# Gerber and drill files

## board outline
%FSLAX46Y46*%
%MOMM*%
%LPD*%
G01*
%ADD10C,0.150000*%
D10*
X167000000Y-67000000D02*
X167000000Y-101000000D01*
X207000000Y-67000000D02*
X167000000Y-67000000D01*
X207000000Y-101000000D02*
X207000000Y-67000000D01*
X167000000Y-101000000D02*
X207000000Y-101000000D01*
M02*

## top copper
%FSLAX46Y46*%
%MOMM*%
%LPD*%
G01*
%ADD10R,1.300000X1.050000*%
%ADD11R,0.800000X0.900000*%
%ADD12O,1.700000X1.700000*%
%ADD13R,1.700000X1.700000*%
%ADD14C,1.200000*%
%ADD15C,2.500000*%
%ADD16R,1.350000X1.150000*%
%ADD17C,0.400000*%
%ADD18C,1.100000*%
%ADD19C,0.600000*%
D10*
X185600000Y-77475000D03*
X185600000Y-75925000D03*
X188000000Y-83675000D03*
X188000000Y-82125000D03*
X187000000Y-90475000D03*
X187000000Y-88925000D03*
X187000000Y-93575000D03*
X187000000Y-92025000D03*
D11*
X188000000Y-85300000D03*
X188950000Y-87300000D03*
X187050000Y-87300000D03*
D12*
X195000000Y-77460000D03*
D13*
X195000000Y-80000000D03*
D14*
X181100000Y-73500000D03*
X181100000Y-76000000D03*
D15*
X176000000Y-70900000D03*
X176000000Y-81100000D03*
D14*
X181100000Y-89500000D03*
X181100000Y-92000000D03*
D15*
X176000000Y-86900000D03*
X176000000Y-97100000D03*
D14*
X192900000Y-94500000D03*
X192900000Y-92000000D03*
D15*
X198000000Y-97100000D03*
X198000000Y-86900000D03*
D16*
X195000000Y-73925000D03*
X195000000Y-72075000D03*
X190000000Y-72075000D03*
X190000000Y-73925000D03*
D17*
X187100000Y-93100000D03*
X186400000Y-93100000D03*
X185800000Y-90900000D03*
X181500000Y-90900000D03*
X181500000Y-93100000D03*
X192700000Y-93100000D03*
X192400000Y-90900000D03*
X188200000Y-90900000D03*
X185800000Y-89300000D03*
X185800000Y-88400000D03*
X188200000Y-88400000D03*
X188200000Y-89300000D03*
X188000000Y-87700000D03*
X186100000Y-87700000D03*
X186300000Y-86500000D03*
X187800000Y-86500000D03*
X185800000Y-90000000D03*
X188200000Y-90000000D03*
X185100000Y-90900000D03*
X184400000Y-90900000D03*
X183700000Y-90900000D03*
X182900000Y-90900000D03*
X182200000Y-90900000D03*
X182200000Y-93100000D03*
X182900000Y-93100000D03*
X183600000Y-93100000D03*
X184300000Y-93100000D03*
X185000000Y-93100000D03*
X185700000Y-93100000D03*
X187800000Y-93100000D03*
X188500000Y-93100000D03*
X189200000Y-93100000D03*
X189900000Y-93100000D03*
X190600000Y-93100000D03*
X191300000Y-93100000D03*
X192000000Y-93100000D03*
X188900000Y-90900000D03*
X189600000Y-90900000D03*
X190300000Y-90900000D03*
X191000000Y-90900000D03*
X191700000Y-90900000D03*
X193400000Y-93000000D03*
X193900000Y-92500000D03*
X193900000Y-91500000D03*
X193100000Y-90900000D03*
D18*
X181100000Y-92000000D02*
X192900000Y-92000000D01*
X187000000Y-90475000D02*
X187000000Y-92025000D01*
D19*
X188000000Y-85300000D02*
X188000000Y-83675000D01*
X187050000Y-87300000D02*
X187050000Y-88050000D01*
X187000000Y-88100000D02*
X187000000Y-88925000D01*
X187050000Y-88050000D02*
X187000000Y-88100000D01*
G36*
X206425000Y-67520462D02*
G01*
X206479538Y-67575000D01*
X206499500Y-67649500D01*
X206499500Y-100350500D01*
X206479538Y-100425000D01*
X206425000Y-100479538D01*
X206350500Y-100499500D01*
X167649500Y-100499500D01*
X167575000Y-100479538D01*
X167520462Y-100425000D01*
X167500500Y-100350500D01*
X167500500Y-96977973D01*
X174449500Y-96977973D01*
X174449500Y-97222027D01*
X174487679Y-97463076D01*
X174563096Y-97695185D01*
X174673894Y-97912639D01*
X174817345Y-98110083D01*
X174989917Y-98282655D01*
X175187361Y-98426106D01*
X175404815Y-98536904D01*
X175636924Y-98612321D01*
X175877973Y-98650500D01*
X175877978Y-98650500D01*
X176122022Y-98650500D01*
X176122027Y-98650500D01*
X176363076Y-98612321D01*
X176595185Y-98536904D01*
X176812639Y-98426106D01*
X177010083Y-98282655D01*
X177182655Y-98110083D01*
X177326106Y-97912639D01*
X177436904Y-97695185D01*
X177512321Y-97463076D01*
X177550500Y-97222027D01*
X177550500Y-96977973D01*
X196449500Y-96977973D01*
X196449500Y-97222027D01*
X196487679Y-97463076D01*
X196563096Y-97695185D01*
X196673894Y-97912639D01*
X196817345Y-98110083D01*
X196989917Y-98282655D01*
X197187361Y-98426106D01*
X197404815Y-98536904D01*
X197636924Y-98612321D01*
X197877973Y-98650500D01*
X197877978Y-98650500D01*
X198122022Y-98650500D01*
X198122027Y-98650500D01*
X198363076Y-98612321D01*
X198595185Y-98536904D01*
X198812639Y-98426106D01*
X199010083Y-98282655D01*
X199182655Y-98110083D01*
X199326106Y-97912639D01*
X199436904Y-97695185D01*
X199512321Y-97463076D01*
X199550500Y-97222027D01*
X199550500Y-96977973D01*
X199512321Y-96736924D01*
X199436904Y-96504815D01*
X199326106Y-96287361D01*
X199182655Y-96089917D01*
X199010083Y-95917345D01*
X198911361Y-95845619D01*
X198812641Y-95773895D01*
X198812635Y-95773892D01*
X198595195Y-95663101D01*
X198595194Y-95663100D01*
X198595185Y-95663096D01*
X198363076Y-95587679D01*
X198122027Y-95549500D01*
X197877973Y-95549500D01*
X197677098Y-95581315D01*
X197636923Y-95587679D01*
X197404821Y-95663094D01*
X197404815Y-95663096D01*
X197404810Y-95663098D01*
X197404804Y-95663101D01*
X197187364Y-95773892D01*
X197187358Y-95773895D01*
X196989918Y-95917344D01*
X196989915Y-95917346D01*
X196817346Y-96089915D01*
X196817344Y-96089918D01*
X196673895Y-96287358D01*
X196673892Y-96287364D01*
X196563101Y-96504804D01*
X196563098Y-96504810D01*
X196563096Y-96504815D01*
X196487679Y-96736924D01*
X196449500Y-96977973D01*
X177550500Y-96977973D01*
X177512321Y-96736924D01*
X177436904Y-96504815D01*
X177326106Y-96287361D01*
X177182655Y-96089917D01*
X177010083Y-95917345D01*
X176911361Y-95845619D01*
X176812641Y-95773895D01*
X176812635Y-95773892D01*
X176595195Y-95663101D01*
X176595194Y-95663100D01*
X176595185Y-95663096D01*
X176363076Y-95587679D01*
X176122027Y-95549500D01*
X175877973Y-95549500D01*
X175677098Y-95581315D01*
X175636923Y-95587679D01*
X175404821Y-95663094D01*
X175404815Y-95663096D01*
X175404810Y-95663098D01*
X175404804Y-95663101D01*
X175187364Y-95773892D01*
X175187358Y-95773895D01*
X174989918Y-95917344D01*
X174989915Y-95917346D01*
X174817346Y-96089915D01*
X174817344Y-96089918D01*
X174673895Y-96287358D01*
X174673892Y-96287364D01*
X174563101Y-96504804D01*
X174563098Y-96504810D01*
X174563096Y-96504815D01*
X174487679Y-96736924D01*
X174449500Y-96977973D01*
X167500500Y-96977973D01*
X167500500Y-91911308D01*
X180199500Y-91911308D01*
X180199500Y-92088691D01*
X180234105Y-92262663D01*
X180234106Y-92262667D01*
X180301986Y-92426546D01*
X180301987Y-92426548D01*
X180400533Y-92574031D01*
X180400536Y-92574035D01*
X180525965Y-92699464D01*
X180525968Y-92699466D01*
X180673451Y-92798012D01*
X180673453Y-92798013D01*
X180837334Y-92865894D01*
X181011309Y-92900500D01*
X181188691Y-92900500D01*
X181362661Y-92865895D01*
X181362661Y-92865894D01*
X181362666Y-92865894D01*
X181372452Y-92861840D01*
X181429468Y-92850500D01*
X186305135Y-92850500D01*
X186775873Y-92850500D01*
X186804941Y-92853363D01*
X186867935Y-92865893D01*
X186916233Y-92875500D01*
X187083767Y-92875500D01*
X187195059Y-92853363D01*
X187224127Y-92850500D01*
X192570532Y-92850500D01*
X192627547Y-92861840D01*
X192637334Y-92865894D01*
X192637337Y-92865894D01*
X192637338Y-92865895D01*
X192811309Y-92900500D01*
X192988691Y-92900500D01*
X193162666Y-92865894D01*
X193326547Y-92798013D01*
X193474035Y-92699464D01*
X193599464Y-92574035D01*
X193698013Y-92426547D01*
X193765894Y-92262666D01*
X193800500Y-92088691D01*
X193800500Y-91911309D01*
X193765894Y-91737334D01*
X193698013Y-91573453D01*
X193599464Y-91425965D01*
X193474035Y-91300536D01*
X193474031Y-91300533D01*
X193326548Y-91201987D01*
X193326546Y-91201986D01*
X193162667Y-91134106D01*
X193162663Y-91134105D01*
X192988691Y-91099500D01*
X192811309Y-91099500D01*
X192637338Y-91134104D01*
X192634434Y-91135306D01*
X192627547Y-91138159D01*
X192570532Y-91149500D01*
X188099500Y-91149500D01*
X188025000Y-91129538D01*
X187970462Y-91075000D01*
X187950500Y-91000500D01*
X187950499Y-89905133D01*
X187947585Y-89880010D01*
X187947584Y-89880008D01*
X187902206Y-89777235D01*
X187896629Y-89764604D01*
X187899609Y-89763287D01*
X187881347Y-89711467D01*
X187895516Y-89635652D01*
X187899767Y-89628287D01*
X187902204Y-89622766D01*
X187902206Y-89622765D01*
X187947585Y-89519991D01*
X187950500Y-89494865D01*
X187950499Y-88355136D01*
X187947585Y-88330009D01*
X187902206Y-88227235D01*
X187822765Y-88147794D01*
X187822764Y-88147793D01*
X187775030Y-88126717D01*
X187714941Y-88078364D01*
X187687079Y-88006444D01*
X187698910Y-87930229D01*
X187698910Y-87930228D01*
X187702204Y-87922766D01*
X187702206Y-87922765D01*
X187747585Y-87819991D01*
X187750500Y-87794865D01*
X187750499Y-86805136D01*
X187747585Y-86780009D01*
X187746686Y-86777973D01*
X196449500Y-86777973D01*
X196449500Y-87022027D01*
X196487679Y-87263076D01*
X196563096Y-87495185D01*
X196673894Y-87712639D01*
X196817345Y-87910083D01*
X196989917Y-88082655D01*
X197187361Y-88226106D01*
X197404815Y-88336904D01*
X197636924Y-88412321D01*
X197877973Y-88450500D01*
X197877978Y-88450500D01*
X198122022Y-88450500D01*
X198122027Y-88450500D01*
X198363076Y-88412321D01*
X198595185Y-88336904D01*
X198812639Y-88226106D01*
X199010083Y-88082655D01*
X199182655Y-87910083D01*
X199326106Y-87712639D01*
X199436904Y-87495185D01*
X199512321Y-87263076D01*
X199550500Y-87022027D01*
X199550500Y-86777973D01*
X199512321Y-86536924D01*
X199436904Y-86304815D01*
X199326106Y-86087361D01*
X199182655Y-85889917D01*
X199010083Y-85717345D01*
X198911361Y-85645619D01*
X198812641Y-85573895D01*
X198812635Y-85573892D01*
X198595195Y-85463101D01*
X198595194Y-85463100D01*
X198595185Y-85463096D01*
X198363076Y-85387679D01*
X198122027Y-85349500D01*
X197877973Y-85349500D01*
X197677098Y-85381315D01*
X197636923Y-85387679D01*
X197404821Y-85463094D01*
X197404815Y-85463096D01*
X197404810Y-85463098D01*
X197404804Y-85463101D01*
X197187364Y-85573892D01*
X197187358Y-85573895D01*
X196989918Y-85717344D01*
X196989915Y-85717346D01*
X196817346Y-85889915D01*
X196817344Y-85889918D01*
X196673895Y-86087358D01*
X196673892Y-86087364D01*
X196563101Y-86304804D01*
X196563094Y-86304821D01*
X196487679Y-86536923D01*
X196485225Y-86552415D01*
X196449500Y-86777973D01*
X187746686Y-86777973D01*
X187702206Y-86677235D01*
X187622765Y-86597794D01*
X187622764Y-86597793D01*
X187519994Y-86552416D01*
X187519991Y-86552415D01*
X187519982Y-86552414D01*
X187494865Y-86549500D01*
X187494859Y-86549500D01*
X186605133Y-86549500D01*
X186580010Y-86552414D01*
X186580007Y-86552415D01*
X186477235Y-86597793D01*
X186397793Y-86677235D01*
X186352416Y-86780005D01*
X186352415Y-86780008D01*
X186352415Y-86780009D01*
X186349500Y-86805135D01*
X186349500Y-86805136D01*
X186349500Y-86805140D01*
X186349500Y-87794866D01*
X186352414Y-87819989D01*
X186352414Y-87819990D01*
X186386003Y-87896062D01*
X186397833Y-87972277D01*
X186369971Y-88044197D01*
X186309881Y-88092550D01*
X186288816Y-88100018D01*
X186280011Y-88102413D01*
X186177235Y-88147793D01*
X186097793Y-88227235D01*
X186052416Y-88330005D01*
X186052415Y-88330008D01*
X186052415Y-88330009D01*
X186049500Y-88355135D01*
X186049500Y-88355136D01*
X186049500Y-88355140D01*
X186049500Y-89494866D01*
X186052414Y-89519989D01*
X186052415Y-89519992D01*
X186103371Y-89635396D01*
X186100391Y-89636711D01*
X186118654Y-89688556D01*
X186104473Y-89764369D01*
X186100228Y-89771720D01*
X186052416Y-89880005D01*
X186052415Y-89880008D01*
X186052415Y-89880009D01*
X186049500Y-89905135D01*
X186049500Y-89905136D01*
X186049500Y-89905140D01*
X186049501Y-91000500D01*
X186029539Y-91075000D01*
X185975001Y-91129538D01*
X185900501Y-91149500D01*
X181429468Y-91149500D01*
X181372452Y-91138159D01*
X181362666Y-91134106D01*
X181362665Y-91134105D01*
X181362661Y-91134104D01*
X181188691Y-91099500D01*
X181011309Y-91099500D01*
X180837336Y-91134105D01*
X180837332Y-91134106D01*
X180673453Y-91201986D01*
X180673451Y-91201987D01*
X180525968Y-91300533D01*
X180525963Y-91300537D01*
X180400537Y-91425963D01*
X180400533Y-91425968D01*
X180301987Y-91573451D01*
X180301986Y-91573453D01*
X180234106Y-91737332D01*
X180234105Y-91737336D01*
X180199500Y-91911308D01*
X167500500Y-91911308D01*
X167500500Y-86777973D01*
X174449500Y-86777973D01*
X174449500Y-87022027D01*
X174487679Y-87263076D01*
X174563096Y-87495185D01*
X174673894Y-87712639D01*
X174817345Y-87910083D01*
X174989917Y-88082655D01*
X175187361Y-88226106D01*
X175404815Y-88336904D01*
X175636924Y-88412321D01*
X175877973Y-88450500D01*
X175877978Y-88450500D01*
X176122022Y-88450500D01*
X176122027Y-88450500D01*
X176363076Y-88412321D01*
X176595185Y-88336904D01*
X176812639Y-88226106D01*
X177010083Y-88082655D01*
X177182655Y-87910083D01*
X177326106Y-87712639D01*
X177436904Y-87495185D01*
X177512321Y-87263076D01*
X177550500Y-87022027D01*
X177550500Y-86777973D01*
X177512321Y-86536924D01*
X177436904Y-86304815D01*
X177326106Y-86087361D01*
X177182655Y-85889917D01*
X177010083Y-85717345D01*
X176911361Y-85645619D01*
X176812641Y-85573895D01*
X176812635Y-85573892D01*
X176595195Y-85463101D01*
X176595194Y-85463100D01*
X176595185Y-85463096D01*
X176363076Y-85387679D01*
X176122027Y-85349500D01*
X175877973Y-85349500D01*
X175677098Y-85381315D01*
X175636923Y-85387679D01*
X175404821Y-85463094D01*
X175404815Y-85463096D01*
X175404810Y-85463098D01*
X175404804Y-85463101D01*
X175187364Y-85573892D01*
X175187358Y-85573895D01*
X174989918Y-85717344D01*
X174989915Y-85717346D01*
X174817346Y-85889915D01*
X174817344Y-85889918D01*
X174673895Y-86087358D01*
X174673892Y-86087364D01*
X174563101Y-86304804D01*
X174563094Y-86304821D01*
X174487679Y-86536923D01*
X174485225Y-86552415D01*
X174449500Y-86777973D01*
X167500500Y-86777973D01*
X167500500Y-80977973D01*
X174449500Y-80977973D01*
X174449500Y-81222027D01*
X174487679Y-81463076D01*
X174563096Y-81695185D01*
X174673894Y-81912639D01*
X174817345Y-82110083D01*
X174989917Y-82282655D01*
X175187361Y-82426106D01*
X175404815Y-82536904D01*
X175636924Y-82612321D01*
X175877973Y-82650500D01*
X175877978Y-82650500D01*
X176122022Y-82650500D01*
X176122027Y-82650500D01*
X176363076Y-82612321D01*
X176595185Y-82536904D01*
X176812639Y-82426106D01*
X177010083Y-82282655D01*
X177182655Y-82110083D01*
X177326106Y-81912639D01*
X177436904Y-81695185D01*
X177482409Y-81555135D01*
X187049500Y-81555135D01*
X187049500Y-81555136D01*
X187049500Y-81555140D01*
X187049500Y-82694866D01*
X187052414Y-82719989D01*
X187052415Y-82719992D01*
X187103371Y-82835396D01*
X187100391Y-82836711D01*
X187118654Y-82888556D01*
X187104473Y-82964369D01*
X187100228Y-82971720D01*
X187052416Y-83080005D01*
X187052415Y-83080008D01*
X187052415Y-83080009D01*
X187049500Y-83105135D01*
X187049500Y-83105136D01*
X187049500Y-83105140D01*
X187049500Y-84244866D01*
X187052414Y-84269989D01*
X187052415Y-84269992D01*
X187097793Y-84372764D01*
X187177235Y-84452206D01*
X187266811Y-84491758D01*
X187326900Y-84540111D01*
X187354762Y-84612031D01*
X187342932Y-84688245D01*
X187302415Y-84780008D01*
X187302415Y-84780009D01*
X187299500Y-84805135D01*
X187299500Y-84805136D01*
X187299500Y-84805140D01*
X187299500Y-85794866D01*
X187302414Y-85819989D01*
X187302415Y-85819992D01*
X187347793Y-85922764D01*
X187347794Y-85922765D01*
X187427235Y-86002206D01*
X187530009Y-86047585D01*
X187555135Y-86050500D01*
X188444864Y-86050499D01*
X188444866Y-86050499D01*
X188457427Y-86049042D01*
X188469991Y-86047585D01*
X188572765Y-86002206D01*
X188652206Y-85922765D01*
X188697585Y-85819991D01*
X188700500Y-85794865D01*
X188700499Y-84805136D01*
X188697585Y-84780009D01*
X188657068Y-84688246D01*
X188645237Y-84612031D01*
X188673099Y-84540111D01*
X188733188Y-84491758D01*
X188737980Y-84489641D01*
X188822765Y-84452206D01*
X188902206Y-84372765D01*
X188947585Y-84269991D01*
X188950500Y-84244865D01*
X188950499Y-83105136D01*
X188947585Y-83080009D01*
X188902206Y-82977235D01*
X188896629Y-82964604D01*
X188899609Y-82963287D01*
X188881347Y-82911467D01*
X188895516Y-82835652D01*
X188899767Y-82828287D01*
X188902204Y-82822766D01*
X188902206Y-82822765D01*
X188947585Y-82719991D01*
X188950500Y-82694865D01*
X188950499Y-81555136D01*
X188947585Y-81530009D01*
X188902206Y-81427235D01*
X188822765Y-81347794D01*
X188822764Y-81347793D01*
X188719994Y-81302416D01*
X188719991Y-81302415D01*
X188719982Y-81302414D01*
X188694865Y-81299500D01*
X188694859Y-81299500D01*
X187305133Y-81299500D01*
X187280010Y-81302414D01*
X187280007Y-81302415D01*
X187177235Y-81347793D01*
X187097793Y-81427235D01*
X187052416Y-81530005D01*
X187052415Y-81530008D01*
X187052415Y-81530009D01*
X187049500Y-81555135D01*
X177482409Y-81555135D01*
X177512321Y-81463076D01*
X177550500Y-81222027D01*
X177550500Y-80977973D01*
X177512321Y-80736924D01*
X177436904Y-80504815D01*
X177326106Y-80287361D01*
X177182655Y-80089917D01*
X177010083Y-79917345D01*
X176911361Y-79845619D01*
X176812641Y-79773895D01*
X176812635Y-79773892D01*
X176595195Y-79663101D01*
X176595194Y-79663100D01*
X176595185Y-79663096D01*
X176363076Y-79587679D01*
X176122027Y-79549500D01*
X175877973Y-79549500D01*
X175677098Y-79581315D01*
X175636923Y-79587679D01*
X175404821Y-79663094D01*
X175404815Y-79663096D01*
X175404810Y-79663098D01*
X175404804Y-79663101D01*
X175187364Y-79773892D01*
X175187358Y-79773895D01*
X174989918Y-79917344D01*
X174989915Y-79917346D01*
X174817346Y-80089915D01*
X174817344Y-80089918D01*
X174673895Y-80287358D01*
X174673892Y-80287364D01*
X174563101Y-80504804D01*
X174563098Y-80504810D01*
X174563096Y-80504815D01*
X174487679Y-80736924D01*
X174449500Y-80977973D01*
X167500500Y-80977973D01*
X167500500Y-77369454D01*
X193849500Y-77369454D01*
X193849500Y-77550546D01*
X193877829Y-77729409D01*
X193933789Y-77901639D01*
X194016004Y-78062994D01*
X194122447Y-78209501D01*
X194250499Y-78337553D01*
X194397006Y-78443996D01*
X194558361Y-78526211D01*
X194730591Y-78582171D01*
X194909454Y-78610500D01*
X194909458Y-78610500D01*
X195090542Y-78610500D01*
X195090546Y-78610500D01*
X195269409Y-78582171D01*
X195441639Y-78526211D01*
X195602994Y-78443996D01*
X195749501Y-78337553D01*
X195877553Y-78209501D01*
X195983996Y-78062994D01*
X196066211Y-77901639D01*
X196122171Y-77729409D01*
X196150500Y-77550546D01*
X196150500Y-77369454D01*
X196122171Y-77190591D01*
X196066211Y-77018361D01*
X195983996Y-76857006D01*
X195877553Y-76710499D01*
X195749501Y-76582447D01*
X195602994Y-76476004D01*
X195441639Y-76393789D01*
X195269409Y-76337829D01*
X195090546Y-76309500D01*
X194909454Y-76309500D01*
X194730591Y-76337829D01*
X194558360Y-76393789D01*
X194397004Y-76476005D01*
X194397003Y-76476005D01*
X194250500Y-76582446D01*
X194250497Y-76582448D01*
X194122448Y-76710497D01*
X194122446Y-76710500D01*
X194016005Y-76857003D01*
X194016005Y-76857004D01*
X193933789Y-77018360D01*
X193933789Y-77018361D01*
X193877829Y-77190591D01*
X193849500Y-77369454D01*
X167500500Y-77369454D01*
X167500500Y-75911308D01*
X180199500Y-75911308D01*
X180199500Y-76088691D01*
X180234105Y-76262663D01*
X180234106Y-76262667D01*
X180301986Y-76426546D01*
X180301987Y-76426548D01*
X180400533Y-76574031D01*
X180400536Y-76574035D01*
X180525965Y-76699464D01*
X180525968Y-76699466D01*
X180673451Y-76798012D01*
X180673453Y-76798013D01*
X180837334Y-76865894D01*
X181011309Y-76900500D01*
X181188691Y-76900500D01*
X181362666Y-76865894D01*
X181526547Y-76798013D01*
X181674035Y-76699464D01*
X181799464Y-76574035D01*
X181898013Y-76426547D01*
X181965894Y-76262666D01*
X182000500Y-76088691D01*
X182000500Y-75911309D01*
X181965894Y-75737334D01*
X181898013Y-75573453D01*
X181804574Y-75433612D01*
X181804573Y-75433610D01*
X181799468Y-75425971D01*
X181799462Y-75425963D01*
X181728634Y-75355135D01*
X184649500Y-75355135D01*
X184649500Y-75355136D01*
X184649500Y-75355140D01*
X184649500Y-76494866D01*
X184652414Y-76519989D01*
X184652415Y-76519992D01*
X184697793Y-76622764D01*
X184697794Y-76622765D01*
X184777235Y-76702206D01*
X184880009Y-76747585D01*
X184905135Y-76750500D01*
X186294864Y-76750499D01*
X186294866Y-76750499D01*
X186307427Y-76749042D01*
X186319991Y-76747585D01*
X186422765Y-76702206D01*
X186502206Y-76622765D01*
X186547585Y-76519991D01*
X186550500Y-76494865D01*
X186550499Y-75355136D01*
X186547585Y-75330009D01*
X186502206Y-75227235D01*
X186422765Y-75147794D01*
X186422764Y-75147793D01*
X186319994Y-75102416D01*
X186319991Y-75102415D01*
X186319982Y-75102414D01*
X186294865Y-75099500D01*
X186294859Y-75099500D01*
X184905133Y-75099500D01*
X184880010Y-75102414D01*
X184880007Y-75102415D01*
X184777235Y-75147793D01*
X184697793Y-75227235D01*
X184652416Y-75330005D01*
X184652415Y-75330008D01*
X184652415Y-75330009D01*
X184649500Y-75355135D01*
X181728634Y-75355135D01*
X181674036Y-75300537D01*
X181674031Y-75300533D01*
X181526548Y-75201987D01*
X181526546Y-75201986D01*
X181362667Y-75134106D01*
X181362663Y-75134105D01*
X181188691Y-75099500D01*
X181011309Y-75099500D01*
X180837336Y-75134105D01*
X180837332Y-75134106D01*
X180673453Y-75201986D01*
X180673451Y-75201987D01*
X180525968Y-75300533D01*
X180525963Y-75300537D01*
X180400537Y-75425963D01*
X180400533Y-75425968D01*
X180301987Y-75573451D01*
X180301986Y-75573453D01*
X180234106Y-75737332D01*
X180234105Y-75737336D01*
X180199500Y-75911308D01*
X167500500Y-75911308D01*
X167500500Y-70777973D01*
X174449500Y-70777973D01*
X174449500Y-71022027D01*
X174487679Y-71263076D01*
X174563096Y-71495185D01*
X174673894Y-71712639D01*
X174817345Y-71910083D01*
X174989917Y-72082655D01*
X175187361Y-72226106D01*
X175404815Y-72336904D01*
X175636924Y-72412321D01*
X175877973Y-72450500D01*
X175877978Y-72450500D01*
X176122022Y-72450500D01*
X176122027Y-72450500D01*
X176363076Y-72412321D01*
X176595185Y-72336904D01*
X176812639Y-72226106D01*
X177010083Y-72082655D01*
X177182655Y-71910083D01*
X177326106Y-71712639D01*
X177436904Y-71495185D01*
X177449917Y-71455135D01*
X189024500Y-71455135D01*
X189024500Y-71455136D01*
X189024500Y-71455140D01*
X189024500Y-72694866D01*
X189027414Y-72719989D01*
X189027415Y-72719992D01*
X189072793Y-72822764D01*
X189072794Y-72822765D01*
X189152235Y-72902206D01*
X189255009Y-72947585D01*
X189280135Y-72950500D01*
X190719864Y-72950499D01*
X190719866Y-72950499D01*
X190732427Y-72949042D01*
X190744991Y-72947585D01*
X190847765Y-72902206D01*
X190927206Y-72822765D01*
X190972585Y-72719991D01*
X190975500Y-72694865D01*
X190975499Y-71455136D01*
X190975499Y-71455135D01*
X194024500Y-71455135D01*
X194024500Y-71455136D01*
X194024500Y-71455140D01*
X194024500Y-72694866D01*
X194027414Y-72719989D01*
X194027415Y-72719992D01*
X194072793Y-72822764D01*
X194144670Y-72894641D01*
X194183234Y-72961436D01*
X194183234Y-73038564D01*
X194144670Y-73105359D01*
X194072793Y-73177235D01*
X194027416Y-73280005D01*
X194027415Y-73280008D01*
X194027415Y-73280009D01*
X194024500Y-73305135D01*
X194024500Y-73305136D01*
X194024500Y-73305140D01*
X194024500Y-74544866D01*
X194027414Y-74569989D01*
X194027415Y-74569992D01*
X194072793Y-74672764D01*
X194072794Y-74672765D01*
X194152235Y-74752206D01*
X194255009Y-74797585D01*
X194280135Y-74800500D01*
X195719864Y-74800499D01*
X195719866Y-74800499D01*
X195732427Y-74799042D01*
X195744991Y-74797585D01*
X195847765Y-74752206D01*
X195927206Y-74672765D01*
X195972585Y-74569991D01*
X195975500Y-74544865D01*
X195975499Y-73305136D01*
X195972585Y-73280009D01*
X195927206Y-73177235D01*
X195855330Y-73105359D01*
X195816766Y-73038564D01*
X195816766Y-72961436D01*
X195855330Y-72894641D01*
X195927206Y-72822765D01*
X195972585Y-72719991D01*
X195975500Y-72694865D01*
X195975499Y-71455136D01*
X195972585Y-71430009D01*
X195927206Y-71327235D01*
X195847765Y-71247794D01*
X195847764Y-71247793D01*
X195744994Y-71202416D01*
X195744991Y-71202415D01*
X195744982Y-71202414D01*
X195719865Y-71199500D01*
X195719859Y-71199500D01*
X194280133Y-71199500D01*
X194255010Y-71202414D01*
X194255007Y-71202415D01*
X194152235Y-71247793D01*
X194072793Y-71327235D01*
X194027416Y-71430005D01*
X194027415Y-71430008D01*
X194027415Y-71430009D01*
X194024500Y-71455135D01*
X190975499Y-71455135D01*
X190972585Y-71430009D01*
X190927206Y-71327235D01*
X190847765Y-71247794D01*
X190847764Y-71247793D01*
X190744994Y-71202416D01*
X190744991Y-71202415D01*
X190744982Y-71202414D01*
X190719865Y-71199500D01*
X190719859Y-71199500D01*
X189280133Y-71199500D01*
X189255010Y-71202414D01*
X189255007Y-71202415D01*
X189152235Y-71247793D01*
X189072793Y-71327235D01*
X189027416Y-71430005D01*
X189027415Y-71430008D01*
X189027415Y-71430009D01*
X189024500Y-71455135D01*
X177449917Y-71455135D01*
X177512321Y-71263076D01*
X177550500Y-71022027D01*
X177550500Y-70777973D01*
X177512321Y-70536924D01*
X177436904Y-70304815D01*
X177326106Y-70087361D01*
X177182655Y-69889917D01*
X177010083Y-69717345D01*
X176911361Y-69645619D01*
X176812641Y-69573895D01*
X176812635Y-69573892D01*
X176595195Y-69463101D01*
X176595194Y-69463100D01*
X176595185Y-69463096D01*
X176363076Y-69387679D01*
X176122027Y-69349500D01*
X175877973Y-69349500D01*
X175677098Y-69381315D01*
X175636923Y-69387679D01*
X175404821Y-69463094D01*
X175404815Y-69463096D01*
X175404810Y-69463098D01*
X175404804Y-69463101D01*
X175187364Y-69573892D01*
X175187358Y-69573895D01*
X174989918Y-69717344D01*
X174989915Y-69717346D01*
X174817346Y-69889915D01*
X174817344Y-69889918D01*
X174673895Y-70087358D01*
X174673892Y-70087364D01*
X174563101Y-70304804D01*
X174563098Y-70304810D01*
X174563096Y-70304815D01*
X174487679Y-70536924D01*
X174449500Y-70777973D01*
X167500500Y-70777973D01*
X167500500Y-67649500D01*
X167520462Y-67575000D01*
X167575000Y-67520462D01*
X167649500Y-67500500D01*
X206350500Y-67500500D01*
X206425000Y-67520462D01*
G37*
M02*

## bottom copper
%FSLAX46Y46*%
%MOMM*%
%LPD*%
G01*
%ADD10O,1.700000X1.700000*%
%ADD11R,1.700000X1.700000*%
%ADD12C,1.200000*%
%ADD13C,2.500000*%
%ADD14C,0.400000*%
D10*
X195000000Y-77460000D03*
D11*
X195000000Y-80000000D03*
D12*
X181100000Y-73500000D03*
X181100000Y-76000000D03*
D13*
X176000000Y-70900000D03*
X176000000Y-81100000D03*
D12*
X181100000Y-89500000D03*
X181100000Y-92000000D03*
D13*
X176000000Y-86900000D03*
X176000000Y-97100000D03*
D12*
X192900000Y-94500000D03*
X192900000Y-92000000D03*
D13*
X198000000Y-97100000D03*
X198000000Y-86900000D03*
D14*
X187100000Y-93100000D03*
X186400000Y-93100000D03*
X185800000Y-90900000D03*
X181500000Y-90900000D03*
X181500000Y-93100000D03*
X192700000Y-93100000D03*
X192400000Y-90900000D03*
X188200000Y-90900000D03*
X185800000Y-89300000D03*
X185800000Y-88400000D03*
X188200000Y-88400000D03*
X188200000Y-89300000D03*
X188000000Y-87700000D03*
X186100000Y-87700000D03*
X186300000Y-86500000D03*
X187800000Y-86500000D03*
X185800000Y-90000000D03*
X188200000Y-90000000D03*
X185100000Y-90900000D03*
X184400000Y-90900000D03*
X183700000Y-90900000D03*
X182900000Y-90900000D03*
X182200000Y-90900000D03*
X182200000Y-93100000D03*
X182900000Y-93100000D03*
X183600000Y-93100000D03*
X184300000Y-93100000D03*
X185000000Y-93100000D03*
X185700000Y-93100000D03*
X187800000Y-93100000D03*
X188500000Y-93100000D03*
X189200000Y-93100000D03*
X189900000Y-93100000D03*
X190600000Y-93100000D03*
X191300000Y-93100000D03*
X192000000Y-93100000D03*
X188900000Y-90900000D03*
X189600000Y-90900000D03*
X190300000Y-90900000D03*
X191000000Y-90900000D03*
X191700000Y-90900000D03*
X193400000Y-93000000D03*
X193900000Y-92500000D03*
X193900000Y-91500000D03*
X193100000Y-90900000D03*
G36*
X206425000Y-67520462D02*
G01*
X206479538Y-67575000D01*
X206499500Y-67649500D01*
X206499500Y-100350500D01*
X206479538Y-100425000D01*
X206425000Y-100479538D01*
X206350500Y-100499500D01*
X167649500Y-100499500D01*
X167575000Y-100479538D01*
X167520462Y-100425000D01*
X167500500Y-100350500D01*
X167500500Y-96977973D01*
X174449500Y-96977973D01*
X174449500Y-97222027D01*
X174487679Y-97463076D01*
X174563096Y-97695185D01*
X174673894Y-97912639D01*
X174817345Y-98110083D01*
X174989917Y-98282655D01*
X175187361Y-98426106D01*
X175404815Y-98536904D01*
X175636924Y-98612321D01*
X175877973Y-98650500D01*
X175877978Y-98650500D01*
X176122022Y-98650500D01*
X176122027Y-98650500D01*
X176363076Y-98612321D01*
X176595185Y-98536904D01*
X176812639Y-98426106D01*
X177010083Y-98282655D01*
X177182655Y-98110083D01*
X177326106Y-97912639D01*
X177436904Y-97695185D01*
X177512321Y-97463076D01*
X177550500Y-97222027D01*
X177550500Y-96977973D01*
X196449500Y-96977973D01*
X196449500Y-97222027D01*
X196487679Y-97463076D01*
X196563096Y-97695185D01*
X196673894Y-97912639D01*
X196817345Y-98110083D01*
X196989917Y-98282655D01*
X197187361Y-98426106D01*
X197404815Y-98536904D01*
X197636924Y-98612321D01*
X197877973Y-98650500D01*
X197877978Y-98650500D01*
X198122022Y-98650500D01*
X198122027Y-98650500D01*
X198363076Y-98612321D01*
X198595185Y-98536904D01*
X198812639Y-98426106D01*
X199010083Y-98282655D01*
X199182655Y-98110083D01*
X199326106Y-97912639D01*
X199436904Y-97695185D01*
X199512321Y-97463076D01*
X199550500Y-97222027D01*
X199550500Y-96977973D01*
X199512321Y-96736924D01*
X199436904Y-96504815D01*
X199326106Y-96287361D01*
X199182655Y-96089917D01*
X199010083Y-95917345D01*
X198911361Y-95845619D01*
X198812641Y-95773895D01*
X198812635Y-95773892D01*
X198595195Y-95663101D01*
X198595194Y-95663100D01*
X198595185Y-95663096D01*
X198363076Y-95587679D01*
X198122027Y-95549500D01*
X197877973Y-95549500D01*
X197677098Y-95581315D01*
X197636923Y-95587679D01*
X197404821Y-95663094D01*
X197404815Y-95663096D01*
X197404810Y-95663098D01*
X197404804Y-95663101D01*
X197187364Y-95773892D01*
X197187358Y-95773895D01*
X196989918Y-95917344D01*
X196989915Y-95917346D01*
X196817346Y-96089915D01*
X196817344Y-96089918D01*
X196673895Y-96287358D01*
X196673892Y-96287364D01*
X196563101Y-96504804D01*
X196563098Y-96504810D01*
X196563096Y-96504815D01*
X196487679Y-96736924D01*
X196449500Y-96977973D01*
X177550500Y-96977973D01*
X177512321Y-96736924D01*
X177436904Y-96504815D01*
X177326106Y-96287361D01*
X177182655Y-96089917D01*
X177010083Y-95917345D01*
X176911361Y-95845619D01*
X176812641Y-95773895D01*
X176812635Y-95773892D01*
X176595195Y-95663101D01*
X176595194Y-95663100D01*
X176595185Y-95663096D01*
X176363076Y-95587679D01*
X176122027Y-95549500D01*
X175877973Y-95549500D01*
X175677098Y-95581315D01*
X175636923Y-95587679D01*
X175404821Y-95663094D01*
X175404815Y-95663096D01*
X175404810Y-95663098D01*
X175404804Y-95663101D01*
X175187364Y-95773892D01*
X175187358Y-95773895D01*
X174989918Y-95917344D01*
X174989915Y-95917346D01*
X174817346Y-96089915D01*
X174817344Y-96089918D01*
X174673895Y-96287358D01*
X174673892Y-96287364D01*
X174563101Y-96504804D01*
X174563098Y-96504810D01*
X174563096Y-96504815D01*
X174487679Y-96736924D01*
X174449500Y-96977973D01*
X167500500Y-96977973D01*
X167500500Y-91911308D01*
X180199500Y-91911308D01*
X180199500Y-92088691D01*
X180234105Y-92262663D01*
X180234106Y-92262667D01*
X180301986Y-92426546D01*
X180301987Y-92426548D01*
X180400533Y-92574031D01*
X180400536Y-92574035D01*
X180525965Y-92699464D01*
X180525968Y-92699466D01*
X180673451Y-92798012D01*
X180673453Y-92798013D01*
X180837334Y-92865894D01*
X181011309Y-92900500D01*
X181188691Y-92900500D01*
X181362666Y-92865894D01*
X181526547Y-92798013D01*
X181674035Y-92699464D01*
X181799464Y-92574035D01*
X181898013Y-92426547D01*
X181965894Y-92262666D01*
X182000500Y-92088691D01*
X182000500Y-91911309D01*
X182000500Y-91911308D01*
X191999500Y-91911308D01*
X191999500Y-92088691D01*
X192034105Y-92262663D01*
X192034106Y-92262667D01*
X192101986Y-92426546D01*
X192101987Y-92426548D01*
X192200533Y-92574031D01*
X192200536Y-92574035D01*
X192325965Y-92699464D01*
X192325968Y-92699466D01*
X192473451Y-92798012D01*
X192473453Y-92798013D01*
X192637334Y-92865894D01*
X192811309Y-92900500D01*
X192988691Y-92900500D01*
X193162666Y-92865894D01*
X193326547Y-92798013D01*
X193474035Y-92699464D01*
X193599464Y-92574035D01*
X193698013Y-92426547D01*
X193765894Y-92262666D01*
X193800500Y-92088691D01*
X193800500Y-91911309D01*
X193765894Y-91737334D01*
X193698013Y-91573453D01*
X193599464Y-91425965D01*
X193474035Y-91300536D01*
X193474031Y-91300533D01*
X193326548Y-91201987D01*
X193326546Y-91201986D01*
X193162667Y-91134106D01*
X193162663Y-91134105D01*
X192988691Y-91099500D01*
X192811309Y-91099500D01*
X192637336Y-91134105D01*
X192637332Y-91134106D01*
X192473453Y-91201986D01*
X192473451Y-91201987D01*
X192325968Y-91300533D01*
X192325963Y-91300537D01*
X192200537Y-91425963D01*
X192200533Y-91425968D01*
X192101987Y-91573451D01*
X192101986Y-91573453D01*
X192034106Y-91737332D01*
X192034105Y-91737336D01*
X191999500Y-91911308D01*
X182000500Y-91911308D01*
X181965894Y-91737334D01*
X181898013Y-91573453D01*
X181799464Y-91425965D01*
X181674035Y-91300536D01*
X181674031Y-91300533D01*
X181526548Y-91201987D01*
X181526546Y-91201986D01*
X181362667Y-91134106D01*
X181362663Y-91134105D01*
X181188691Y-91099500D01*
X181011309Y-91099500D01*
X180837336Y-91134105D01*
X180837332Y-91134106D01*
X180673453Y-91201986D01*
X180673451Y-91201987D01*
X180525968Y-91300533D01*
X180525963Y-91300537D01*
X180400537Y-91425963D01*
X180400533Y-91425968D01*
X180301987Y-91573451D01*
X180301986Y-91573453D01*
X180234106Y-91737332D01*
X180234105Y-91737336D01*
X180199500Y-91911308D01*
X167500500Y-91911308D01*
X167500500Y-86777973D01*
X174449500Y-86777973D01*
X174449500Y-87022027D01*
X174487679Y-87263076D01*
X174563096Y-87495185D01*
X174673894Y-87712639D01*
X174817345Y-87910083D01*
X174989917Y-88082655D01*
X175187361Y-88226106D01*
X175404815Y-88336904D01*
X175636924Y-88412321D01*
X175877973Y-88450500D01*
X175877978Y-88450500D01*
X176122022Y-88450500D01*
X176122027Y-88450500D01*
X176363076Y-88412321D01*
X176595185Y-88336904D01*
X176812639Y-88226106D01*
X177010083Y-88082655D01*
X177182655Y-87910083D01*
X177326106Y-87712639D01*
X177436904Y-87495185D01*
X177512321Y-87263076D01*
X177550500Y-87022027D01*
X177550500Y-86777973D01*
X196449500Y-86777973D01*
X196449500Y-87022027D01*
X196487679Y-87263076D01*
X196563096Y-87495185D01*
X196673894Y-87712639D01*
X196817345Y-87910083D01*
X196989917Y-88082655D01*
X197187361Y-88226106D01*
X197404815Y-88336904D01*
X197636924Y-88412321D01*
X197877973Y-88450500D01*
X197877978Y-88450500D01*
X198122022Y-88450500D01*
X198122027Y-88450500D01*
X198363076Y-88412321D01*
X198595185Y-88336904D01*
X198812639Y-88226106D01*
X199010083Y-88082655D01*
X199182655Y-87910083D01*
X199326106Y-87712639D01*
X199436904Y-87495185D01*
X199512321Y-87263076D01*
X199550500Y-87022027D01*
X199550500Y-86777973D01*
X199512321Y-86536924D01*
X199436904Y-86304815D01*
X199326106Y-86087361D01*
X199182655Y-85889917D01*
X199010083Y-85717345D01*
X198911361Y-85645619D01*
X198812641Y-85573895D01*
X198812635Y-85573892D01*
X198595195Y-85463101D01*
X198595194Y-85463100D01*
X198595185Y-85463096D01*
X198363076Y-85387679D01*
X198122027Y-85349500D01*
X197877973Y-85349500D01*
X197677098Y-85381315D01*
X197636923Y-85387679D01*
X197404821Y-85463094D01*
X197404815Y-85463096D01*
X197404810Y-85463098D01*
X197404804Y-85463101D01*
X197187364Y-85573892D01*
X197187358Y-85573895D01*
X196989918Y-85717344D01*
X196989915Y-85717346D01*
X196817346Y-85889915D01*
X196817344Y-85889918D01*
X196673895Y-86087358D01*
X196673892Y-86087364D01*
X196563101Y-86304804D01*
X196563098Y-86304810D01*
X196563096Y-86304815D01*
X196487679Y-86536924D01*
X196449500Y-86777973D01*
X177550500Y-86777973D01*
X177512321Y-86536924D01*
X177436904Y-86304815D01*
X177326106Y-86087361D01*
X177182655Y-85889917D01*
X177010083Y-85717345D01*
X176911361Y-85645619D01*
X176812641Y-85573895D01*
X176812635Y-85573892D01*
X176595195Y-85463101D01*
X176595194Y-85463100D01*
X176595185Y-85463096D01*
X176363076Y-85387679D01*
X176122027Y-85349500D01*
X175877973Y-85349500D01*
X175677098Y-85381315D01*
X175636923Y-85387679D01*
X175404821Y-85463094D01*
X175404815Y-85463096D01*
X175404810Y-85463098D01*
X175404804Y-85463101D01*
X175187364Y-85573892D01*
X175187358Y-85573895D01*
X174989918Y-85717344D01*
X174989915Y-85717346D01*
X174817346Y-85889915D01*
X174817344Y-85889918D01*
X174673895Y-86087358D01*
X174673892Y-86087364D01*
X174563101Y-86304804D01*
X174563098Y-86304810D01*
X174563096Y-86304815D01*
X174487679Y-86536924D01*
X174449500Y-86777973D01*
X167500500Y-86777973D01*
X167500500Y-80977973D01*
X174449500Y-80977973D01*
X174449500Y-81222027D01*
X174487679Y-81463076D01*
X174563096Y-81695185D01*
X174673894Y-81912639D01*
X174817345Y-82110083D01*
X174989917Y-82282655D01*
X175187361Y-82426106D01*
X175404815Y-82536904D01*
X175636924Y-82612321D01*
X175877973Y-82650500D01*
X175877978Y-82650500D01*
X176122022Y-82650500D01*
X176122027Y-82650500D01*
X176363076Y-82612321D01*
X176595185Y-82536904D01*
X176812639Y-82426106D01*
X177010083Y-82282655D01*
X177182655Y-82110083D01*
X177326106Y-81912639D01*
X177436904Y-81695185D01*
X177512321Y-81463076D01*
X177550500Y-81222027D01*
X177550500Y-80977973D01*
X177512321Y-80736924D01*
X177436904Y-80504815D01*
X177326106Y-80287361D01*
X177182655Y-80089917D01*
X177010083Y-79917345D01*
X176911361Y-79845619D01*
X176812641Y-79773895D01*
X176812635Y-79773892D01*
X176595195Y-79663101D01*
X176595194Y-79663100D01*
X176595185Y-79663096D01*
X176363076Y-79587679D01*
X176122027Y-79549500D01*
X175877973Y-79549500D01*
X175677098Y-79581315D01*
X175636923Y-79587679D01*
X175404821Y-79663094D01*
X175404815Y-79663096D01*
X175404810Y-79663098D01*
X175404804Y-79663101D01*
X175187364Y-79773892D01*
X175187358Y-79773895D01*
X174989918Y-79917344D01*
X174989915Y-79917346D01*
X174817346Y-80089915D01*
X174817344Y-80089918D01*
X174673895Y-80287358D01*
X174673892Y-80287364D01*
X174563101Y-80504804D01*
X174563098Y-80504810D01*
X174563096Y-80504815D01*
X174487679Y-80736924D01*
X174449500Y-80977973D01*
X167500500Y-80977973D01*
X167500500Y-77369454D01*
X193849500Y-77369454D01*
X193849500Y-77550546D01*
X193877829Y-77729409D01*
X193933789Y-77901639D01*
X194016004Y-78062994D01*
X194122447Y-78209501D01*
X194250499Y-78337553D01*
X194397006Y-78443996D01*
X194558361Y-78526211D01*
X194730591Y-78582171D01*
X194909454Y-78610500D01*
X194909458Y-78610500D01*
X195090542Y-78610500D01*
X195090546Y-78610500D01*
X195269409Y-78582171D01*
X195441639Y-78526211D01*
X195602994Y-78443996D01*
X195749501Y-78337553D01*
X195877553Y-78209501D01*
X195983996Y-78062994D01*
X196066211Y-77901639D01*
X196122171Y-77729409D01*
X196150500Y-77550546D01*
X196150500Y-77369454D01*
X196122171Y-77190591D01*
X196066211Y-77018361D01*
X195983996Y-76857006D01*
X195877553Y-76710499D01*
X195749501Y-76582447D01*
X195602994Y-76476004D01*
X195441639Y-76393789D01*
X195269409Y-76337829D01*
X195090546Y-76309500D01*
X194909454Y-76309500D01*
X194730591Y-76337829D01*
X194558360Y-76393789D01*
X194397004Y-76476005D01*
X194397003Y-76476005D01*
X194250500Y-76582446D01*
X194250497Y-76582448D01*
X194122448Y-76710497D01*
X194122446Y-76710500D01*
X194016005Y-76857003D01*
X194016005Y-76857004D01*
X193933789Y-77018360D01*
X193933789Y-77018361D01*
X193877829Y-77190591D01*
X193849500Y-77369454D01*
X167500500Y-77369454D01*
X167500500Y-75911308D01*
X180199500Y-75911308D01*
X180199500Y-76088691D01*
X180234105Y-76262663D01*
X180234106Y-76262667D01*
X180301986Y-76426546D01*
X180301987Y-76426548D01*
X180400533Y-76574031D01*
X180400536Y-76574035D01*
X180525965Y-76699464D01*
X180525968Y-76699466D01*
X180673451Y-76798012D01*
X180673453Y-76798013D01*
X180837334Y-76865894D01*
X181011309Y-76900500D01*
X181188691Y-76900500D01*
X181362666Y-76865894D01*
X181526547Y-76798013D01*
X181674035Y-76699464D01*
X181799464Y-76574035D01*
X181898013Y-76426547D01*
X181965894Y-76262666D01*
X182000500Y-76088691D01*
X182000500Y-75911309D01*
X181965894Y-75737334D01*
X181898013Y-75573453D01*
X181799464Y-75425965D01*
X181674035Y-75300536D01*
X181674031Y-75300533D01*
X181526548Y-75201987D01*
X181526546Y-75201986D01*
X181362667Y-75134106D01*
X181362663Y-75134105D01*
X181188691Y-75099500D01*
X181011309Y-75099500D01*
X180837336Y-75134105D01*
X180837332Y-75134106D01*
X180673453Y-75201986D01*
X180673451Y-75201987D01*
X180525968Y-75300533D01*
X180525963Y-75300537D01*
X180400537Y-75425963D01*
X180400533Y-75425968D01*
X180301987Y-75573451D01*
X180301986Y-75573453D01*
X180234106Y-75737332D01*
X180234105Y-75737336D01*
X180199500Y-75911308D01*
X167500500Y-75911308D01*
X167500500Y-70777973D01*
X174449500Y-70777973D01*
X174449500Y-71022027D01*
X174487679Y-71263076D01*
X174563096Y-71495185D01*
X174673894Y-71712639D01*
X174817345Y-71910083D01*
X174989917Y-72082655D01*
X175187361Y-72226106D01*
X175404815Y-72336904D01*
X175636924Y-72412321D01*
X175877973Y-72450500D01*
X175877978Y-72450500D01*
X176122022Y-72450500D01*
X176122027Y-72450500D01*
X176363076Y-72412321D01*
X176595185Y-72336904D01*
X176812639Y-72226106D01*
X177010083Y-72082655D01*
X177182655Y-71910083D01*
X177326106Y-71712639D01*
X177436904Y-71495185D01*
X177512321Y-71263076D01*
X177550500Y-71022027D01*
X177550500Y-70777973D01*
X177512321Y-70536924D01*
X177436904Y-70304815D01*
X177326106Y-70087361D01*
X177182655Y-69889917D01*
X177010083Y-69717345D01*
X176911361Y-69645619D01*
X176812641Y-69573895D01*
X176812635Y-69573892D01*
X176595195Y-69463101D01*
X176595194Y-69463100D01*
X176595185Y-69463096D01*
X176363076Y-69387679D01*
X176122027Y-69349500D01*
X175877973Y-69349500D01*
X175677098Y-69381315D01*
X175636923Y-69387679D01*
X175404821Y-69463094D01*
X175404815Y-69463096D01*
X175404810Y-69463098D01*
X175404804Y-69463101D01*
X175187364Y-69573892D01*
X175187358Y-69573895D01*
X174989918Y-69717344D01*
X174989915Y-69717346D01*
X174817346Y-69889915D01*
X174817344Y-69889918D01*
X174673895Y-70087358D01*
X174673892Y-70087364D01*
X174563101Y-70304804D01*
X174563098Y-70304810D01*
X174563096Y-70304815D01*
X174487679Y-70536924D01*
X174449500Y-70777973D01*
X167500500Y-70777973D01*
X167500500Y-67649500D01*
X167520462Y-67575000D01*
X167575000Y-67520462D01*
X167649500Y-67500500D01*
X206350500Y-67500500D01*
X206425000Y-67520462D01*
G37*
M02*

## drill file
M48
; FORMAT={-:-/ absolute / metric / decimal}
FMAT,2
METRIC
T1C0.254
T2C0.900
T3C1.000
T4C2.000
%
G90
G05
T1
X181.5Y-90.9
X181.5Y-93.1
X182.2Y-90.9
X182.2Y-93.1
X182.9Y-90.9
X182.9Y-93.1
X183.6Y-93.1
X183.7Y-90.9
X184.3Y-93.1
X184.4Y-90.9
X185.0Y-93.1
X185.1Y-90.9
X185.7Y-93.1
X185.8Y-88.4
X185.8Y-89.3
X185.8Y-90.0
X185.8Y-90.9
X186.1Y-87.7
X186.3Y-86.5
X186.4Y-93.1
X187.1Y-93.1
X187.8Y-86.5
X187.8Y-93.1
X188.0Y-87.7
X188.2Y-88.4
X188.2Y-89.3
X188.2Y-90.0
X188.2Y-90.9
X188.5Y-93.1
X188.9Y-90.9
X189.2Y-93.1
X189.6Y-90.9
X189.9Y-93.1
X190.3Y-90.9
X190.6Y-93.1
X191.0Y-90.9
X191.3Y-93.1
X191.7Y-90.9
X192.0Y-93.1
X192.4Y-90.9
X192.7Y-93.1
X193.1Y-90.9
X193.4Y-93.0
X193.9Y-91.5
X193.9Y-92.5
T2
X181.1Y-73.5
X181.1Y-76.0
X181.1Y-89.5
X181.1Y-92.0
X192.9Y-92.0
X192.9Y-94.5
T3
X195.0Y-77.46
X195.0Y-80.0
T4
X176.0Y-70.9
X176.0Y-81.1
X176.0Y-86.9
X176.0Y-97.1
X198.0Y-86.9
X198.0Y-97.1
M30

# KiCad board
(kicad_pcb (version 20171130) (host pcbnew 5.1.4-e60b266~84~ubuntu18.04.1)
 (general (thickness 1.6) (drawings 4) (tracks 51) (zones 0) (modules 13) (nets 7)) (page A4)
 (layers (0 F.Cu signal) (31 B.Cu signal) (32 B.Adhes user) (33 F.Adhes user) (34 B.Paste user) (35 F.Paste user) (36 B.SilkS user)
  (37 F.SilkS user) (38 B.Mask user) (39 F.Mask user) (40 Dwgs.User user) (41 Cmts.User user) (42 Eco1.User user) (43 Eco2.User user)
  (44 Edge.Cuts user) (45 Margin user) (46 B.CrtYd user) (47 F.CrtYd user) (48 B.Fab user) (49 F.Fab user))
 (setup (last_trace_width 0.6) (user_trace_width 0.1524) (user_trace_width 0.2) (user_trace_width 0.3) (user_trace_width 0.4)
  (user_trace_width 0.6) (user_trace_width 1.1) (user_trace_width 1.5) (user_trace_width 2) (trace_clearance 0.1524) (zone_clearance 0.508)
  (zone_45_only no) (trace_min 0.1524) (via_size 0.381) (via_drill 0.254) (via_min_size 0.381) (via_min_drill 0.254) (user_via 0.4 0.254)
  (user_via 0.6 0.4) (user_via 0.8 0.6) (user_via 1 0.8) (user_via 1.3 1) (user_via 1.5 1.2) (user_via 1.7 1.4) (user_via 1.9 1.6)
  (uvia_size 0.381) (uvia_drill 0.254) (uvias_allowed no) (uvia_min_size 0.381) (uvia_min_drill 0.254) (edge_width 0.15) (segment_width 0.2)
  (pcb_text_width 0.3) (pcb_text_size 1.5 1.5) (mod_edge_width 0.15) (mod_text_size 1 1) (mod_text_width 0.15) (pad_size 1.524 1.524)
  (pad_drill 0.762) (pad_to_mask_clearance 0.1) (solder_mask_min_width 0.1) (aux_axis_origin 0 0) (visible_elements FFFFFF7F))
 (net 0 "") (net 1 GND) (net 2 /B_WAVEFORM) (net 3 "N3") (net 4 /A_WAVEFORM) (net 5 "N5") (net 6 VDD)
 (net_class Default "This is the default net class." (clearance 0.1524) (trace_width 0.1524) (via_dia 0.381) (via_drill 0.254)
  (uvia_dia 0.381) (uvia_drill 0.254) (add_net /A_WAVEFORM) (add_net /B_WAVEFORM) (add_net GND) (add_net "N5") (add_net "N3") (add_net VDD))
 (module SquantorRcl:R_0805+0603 (layer F.Cu) (at 185.6 76.7 270)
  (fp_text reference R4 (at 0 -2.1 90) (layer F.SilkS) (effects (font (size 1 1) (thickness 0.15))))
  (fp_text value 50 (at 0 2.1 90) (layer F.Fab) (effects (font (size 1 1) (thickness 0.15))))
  (pad 2 smd rect (at 0.775 0 270) (size 1.05 1.3) (layers F.Cu F.Paste F.Mask) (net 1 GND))
  (pad 1 smd rect (at -0.775 0 270) (size 1.05 1.3) (layers F.Cu F.Paste F.Mask) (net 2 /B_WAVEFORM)))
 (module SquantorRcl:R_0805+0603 (layer F.Cu) (at 188 82.9 270)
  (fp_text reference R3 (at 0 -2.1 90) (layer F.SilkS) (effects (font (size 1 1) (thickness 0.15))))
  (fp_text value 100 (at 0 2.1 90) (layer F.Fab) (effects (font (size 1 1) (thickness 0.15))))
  (pad 2 smd rect (at 0.775 0 270) (size 1.05 1.3) (layers F.Cu F.Paste F.Mask) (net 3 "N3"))
  (pad 1 smd rect (at -0.775 0 270) (size 1.05 1.3) (layers F.Cu F.Paste F.Mask) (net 2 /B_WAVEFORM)))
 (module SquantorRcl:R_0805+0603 (layer F.Cu) (at 187 89.7 270)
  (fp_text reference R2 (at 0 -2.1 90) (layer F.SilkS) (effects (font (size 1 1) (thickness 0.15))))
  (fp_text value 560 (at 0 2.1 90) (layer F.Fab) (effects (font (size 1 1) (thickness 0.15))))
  (pad 2 smd rect (at 0.775 0 270) (size 1.05 1.3) (layers F.Cu F.Paste F.Mask) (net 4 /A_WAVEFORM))
  (pad 1 smd rect (at -0.775 0 270) (size 1.05 1.3) (layers F.Cu F.Paste F.Mask) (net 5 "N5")))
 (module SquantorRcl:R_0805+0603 (layer F.Cu) (at 187 92.8 270)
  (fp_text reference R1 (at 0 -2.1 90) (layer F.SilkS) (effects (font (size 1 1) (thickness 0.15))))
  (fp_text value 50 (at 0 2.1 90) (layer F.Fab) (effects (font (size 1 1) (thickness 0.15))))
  (pad 2 smd rect (at 0.775 0 270) (size 1.05 1.3) (layers F.Cu F.Paste F.Mask) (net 1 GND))
  (pad 1 smd rect (at -0.775 0 270) (size 1.05 1.3) (layers F.Cu F.Paste F.Mask) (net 4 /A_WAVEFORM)))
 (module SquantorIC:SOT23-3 (layer F.Cu) (at 188 86.3)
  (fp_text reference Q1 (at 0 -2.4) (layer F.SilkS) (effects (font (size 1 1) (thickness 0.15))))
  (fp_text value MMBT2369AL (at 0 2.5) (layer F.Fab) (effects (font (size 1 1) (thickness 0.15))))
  (pad 3 smd rect (at 0 -1) (size 0.8 0.9) (layers F.Cu F.Paste F.Mask) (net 3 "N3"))
  (pad 2 smd rect (at 0.95 1) (size 0.8 0.9) (layers F.Cu F.Paste F.Mask) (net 1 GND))
  (pad 1 smd rect (at -0.95 1) (size 0.8 0.9) (layers F.Cu F.Paste F.Mask) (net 5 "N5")))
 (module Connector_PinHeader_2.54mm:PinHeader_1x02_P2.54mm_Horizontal (layer B.Cu) (at 195 80)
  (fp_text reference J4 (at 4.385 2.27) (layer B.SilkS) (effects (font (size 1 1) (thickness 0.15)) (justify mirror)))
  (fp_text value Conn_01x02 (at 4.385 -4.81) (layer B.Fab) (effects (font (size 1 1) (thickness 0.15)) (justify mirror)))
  (pad 2 thru_hole oval (at 0 -2.54) (size 1.7 1.7) (drill 1) (layers *.Cu *.Mask) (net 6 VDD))
  (pad 1 thru_hole rect (at 0 0) (size 1.7 1.7) (drill 1) (layers *.Cu *.Mask) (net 1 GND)))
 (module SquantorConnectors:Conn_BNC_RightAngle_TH (layer B.Cu) (at 176 76 270)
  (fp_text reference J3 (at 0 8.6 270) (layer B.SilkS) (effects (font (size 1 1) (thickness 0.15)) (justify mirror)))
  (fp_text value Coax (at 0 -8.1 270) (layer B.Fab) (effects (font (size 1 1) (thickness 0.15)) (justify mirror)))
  (pad G thru_hole circle (at -2.5 -5.1 270) (size 1.2 1.2) (drill 0.9) (layers *.Cu *.Mask) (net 1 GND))
  (pad S thru_hole circle (at 0 -5.1 270) (size 1.2 1.2) (drill 0.9) (layers *.Cu *.Mask) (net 2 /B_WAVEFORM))
  (pad mount thru_hole circle (at -5.1 0 270) (size 2.5 2.5) (drill 2) (layers *.Cu *.Mask))
  (pad mount thru_hole circle (at 5.1 0 270) (size 2.5 2.5) (drill 2) (layers *.Cu *.Mask)))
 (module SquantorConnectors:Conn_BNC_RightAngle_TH (layer B.Cu) (at 176 92 270)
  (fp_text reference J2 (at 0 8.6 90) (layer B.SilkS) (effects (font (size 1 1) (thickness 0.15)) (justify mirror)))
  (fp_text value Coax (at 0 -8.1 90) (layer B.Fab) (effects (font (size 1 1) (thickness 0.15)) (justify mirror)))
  (pad G thru_hole circle (at -2.5 -5.1 270) (size 1.2 1.2) (drill 0.9) (layers *.Cu *.Mask) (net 1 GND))
  (pad S thru_hole circle (at 0 -5.1 270) (size 1.2 1.2) (drill 0.9) (layers *.Cu *.Mask) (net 4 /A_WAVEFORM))
  (pad mount thru_hole circle (at -5.1 0 270) (size 2.5 2.5) (drill 2) (layers *.Cu *.Mask))
  (pad mount thru_hole circle (at 5.1 0 270) (size 2.5 2.5) (drill 2) (layers *.Cu *.Mask)))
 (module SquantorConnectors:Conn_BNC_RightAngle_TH (layer B.Cu) (at 198 92 90)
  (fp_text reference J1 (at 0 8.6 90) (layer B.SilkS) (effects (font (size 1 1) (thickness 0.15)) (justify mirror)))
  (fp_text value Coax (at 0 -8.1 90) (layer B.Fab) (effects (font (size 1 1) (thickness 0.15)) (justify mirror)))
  (pad G thru_hole circle (at -2.5 -5.1 90) (size 1.2 1.2) (drill 0.9) (layers *.Cu *.Mask) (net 1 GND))
  (pad S thru_hole circle (at 0 -5.1 90) (size 1.2 1.2) (drill 0.9) (layers *.Cu *.Mask) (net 4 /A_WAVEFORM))
  (pad mount thru_hole circle (at -5.1 0 90) (size 2.5 2.5) (drill 2) (layers *.Cu *.Mask))
  (pad mount thru_hole circle (at 5.1 0 90) (size 2.5 2.5) (drill 2) (layers *.Cu *.Mask)))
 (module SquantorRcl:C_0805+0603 (layer F.Cu) (at 195 73 90)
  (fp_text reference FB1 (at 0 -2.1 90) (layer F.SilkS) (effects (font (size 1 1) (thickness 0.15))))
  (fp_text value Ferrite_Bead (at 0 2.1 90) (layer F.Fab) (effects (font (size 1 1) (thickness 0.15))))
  (pad 1 smd rect (at -0.925 0 90) (size 1.15 1.35) (layers F.Cu F.Paste F.Mask) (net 6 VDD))
  (pad 2 smd rect (at 0.925 0 90) (size 1.15 1.35) (layers F.Cu F.Paste F.Mask) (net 2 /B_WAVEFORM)))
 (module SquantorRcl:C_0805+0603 (layer F.Cu) (at 190 73 270)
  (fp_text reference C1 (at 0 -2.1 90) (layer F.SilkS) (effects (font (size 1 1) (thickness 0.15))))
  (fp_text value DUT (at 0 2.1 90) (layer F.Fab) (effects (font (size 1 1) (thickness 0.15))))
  (pad 1 smd rect (at -0.925 0 270) (size 1.15 1.35) (layers F.Cu F.Paste F.Mask) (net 2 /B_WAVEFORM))
  (pad 2 smd rect (at 0.925 0 270) (size 1.15 1.35) (layers F.Cu F.Paste F.Mask) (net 1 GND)))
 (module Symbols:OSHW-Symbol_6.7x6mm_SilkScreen (layer B.Cu) (at 188.5 74 180)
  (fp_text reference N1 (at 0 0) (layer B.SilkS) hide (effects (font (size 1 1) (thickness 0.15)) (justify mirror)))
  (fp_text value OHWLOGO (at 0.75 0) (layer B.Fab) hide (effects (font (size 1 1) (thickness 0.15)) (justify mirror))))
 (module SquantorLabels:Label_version (layer B.Cu) (at 188 78)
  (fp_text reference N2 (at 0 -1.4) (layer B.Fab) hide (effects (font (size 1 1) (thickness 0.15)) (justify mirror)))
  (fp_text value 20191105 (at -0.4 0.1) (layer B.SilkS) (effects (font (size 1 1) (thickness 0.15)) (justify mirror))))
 (gr_line (start 167 67) (end 167 101) (layer Edge.Cuts) (width 0.15))
 (gr_line (start 207 67) (end 167 67) (layer Edge.Cuts) (width 0.15))
 (gr_line (start 207 101) (end 207 67) (layer Edge.Cuts) (width 0.15))
 (gr_line (start 167 101) (end 207 101) (layer Edge.Cuts) (width 0.15))
 (via (at 187.1 93.1) (size 0.4) (drill 0.254) (layers F.Cu B.Cu) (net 1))
 (via (at 186.4 93.1) (size 0.4) (drill 0.254) (layers F.Cu B.Cu) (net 1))
 (via (at 185.8 90.9) (size 0.4) (drill 0.254) (layers F.Cu B.Cu) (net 1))
 (via (at 181.5 90.9) (size 0.4) (drill 0.254) (layers F.Cu B.Cu) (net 1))
 (via (at 181.5 93.1) (size 0.4) (drill 0.254) (layers F.Cu B.Cu) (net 1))
 (via (at 192.7 93.1) (size 0.4) (drill 0.254) (layers F.Cu B.Cu) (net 1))
 (via (at 192.4 90.9) (size 0.4) (drill 0.254) (layers F.Cu B.Cu) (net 1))
 (via (at 188.2 90.9) (size 0.4) (drill 0.254) (layers F.Cu B.Cu) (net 1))
 (via (at 185.8 89.3) (size 0.4) (drill 0.254) (layers F.Cu B.Cu) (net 1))
 (via (at 185.8 88.4) (size 0.4) (drill 0.254) (layers F.Cu B.Cu) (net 1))
 (via (at 188.2 88.4) (size 0.4) (drill 0.254) (layers F.Cu B.Cu) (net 1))
 (via (at 188.2 89.3) (size 0.4) (drill 0.254) (layers F.Cu B.Cu) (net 1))
 (via (at 188 87.7) (size 0.4) (drill 0.254) (layers F.Cu B.Cu) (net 1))
 (via (at 186.1 87.7) (size 0.4) (drill 0.254) (layers F.Cu B.Cu) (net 1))
 (via (at 186.3 86.5) (size 0.4) (drill 0.254) (layers F.Cu B.Cu) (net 1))
 (via (at 187.8 86.5) (size 0.4) (drill 0.254) (layers F.Cu B.Cu) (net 1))
 (via (at 185.8 90) (size 0.4) (drill 0.254) (layers F.Cu B.Cu) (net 1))
 (via (at 188.2 90) (size 0.4) (drill 0.254) (layers F.Cu B.Cu) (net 1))
 (via (at 185.1 90.9) (size 0.4) (drill 0.254) (layers F.Cu B.Cu) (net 1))
 (via (at 184.4 90.9) (size 0.4) (drill 0.254) (layers F.Cu B.Cu) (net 1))
 (via (at 183.7 90.9) (size 0.4) (drill 0.254) (layers F.Cu B.Cu) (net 1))
 (via (at 182.9 90.9) (size 0.4) (drill 0.254) (layers F.Cu B.Cu) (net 1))
 (via (at 182.2 90.9) (size 0.4) (drill 0.254) (layers F.Cu B.Cu) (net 1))
 (via (at 182.2 93.1) (size 0.4) (drill 0.254) (layers F.Cu B.Cu) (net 1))
 (via (at 182.9 93.1) (size 0.4) (drill 0.254) (layers F.Cu B.Cu) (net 1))
 (via (at 183.6 93.1) (size 0.4) (drill 0.254) (layers F.Cu B.Cu) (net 1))
 (via (at 184.3 93.1) (size 0.4) (drill 0.254) (layers F.Cu B.Cu) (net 1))
 (via (at 185 93.1) (size 0.4) (drill 0.254) (layers F.Cu B.Cu) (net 1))
 (via (at 185.7 93.1) (size 0.4) (drill 0.254) (layers F.Cu B.Cu) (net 1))
 (via (at 187.8 93.1) (size 0.4) (drill 0.254) (layers F.Cu B.Cu) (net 1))
 (via (at 188.5 93.1) (size 0.4) (drill 0.254) (layers F.Cu B.Cu) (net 1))
 (via (at 189.2 93.1) (size 0.4) (drill 0.254) (layers F.Cu B.Cu) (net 1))
 (via (at 189.9 93.1) (size 0.4) (drill 0.254) (layers F.Cu B.Cu) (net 1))
 (via (at 190.6 93.1) (size 0.4) (drill 0.254) (layers F.Cu B.Cu) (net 1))
 (via (at 191.3 93.1) (size 0.4) (drill 0.254) (layers F.Cu B.Cu) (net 1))
 (via (at 192 93.1) (size 0.4) (drill 0.254) (layers F.Cu B.Cu) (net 1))
 (via (at 188.9 90.9) (size 0.4) (drill 0.254) (layers F.Cu B.Cu) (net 1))
 (via (at 189.6 90.9) (size 0.4) (drill 0.254) (layers F.Cu B.Cu) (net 1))
 (via (at 190.3 90.9) (size 0.4) (drill 0.254) (layers F.Cu B.Cu) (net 1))
 (via (at 191 90.9) (size 0.4) (drill 0.254) (layers F.Cu B.Cu) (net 1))
 (via (at 191.7 90.9) (size 0.4) (drill 0.254) (layers F.Cu B.Cu) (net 1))
 (via (at 193.4 93) (size 0.4) (drill 0.254) (layers F.Cu B.Cu) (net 1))
 (via (at 193.9 92.5) (size 0.4) (drill 0.254) (layers F.Cu B.Cu) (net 1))
 (via (at 193.9 91.5) (size 0.4) (drill 0.254) (layers F.Cu B.Cu) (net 1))
 (via (at 193.1 90.9) (size 0.4) (drill 0.254) (layers F.Cu B.Cu) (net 1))
 (segment (start 181.1 92) (end 192.9 92) (width 1.1) (layer F.Cu) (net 4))
 (segment (start 187 90.475) (end 187 92.025) (width 1.1) (layer F.Cu) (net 4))
 (segment (start 188 85.3) (end 188 83.675) (width 0.6) (layer F.Cu) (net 3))
 (segment (start 187.05 87.3) (end 187.05 88.05) (width 0.6) (layer F.Cu) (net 5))
 (segment (start 187 88.1) (end 187 88.925) (width 0.6) (layer F.Cu) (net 5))
 (segment (start 187.05 88.05) (end 187 88.1) (width 0.6) (layer F.Cu) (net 5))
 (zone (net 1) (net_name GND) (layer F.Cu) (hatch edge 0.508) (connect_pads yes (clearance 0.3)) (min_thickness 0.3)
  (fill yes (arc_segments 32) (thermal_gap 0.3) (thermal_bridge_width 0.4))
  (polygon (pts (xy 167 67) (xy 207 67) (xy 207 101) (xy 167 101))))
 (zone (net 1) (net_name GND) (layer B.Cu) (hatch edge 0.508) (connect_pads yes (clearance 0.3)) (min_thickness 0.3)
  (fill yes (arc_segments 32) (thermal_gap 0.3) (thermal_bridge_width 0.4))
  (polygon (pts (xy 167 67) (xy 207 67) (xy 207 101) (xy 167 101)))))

